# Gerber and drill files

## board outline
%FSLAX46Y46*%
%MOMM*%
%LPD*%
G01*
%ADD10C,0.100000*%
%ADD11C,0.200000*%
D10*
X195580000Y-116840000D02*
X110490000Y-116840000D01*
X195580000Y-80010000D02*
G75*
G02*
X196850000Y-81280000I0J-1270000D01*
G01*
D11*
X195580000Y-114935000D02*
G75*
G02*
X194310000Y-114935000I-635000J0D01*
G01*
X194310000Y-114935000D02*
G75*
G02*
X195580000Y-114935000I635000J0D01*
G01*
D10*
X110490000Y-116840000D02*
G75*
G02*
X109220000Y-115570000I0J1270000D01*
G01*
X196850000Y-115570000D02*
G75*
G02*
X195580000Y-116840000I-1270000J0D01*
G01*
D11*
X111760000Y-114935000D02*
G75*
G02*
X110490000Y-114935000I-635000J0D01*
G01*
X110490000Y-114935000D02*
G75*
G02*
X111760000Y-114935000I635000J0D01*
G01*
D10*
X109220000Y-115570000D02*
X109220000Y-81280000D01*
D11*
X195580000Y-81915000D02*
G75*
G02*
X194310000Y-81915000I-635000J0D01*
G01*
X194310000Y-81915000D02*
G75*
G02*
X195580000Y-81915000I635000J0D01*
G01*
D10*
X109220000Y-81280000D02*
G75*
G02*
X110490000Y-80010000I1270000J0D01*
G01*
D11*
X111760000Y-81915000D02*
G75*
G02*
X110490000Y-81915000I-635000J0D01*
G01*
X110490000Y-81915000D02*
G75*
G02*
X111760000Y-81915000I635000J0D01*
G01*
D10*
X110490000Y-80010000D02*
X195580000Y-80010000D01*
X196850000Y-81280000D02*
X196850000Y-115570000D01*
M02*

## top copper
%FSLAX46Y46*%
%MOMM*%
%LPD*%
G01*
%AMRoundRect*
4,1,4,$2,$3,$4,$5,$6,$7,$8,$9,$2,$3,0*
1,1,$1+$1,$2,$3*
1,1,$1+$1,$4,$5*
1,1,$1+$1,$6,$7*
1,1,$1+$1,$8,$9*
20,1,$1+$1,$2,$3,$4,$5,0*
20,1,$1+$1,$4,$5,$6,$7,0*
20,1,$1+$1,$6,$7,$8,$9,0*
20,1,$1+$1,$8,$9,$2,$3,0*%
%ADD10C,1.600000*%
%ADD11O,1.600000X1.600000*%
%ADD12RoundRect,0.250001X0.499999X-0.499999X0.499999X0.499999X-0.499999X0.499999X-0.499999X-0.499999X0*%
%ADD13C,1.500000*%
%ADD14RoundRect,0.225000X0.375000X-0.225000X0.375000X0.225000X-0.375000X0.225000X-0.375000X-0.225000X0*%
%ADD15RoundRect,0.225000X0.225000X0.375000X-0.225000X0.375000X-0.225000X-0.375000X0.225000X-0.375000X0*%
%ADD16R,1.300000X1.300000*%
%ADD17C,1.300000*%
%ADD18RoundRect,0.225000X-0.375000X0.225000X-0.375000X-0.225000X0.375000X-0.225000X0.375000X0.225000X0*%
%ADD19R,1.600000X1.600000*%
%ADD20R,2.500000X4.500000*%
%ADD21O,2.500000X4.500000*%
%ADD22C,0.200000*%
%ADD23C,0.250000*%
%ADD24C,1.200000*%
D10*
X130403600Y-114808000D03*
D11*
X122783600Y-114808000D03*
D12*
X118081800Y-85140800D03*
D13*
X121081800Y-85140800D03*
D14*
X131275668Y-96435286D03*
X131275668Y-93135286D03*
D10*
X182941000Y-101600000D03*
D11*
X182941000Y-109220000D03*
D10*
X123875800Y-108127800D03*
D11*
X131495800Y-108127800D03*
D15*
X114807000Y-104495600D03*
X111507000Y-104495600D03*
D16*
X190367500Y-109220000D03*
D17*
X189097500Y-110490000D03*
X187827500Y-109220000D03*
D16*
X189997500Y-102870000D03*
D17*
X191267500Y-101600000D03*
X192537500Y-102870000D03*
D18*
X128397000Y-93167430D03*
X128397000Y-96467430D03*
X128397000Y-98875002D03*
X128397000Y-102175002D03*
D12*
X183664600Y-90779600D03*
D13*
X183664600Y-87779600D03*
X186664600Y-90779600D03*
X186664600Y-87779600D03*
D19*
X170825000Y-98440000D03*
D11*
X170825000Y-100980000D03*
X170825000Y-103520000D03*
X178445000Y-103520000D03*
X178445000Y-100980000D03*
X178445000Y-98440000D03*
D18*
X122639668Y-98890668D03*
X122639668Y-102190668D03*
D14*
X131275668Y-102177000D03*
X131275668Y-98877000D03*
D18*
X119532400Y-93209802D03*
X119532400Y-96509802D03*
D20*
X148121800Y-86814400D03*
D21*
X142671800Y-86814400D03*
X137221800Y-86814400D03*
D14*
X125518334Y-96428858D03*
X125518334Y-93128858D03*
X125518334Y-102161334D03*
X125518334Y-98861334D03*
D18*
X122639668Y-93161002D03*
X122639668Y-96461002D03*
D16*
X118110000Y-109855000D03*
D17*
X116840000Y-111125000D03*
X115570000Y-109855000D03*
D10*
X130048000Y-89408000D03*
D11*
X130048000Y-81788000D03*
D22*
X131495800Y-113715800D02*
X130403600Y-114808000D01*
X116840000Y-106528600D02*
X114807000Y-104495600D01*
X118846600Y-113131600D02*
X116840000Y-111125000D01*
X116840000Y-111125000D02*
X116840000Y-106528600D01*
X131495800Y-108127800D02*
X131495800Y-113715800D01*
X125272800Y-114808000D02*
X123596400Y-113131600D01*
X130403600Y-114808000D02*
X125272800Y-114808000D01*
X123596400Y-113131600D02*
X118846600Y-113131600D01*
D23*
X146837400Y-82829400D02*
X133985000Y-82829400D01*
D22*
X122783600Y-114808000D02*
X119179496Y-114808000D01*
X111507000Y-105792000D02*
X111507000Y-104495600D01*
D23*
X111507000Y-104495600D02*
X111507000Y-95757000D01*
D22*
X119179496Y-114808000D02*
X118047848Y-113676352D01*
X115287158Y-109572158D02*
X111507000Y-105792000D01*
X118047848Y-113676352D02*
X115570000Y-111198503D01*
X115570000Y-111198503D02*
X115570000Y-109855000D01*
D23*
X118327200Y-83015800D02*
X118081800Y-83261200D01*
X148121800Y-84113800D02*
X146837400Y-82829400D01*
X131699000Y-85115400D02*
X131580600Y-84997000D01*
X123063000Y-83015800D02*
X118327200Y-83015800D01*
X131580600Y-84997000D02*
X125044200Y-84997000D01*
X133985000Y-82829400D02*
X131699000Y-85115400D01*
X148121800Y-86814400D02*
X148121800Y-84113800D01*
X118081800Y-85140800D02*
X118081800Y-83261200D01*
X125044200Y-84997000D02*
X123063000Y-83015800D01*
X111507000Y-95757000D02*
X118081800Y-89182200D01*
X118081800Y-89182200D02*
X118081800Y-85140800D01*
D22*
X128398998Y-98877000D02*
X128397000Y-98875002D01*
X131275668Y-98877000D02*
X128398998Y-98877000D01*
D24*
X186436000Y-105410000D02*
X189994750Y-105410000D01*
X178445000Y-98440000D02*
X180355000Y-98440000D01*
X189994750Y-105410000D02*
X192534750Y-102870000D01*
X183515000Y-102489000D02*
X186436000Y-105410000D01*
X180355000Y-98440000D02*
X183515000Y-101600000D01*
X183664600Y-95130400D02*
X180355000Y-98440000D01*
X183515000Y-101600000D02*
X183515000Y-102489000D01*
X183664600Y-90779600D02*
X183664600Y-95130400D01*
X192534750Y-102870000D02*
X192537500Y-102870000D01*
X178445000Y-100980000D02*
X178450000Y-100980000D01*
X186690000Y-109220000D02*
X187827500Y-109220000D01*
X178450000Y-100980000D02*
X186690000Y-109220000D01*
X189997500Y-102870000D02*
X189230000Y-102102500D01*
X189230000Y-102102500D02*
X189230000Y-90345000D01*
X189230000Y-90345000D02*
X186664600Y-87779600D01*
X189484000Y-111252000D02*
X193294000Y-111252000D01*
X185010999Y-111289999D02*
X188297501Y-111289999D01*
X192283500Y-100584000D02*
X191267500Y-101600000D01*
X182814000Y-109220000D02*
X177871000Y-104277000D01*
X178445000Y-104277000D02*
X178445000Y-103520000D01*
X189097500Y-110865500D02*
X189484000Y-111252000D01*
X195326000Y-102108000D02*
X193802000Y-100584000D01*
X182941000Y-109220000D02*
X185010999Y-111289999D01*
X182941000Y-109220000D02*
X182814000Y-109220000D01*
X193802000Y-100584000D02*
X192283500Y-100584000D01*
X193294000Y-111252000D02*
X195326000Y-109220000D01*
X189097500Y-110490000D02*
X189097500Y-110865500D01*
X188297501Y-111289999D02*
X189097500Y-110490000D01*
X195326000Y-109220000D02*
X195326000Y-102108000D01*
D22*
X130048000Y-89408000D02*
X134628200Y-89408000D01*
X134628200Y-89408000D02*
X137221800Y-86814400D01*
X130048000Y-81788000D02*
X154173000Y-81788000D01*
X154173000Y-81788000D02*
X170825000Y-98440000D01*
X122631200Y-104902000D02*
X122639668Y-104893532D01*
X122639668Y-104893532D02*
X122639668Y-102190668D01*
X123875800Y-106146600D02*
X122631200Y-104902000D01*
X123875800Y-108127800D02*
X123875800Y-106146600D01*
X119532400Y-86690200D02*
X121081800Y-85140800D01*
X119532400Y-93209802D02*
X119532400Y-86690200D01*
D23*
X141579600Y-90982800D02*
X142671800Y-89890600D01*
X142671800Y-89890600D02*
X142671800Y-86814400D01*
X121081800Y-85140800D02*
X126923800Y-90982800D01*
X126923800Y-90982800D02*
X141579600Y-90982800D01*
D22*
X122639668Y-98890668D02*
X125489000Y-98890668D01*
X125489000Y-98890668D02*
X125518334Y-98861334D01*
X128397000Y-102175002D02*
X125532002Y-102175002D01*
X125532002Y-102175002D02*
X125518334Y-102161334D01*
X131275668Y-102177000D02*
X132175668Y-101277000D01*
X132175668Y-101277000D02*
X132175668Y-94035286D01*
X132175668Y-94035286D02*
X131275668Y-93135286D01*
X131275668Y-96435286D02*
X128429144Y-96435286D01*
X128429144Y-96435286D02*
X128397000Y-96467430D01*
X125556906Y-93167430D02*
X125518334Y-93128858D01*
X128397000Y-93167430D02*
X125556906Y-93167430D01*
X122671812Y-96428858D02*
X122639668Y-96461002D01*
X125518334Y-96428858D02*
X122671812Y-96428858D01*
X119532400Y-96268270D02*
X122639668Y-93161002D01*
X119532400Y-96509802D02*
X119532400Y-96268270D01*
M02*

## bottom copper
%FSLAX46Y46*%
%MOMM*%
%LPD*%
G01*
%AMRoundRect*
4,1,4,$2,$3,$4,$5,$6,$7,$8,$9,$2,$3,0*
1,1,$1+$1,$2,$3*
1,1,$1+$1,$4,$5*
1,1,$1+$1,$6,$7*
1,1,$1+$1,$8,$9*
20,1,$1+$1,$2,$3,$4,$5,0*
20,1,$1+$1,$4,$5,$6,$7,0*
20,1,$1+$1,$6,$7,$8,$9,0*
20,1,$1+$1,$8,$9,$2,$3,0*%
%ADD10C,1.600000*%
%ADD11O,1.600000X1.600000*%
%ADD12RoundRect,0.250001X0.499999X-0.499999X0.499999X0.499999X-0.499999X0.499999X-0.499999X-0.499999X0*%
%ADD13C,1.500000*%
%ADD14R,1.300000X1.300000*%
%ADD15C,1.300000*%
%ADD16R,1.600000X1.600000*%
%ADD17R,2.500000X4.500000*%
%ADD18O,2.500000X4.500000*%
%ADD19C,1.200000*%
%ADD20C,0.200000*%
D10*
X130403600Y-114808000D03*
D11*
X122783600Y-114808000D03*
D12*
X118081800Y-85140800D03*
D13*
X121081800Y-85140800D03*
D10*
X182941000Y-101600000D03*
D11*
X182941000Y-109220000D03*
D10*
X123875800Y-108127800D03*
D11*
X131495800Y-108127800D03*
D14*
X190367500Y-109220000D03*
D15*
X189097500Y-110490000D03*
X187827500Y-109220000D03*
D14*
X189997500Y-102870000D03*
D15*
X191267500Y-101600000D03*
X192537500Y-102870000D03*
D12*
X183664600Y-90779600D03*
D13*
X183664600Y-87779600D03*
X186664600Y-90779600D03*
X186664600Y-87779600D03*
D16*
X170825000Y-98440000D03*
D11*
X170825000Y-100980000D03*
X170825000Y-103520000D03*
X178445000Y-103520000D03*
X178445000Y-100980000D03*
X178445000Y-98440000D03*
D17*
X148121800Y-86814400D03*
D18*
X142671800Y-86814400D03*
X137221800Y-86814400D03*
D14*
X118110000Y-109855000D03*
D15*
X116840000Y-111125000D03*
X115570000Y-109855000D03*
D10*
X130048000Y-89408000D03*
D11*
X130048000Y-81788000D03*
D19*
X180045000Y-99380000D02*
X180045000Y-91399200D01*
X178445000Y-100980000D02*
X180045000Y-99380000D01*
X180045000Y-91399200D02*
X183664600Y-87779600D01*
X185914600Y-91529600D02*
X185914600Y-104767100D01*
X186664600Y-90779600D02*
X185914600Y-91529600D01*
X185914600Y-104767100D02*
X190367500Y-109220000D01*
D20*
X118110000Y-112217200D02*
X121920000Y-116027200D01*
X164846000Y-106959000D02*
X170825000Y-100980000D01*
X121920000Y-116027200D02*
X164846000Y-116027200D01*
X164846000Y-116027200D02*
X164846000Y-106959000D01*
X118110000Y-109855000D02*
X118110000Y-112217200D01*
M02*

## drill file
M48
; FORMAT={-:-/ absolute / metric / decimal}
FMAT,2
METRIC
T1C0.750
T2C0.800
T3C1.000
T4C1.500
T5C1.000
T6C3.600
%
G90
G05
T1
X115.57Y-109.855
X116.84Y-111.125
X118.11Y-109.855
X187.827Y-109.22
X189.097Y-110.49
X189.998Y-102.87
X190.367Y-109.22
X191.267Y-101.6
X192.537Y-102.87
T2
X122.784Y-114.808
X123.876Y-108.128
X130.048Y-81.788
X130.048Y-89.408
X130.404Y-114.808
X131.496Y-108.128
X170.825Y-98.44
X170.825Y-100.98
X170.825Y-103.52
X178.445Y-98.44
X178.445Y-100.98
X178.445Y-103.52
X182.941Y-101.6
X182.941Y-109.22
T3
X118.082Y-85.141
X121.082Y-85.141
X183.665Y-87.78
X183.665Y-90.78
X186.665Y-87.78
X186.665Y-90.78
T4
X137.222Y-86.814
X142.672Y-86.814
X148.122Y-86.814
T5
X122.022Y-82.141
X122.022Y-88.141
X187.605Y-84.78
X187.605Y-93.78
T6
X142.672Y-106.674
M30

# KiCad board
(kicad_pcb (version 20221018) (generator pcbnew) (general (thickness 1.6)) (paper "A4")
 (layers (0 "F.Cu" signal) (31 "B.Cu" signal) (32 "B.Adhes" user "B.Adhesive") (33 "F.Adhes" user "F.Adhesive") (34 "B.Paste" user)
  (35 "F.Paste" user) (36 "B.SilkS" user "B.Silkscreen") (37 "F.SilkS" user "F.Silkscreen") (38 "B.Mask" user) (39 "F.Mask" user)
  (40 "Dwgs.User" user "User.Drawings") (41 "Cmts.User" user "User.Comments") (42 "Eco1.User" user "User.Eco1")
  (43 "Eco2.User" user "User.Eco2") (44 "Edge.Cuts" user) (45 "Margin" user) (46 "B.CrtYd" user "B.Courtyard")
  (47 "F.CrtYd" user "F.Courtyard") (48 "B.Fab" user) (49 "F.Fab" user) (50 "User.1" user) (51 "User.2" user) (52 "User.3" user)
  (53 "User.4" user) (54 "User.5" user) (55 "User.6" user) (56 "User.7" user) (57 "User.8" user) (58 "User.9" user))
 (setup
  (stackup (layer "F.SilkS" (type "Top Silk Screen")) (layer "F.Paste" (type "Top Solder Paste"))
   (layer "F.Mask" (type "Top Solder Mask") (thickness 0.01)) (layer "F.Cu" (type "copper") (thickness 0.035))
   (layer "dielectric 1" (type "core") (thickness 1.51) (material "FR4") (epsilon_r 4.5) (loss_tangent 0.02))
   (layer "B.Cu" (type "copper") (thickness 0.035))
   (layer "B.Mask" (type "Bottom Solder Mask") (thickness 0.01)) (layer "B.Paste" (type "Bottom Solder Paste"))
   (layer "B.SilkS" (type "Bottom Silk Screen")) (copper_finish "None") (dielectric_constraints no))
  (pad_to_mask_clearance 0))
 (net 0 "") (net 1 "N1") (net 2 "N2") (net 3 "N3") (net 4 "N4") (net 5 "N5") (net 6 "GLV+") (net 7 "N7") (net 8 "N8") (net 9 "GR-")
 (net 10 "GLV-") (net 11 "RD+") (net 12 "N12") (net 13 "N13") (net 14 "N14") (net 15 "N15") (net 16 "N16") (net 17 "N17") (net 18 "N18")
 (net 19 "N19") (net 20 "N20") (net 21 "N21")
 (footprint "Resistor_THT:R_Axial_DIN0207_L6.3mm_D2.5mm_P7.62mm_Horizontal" (layer "F.Cu") (at 130.4036 114.808 180)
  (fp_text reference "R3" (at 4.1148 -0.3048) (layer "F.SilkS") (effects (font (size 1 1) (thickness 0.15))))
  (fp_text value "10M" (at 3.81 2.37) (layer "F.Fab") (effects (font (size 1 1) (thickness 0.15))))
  (pad "1" thru_hole circle (at 0 0 180) (size 1.6 1.6) (drill 0.8) (layers "*.Cu" "*.Mask") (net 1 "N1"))
  (pad "2" thru_hole oval (at 7.62 0 180) (size 1.6 1.6) (drill 0.8) (layers "*.Cu" "*.Mask") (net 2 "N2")))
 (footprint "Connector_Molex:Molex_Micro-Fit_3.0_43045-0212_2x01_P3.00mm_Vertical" (layer "F.Cu") (at 118.0818 85.1408 90)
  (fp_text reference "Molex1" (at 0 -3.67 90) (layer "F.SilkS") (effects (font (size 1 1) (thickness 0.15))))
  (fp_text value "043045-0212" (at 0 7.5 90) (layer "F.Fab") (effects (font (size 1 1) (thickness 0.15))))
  (pad "" np_thru_hole circle (at -3 3.94 90) (size 1 1) (drill 1) (layers "*.Cu" "*.Mask"))
  (pad "" np_thru_hole circle (at 3 3.94 90) (size 1 1) (drill 1) (layers "*.Cu" "*.Mask"))
  (pad "1" thru_hole roundrect (at 0 0 90) (size 1.5 1.5) (drill 1) (layers "*.Cu" "*.Mask") (roundrect_rratio 0.166667) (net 2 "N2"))
  (pad "2" thru_hole circle (at 0 3 90) (size 1.5 1.5) (drill 1) (layers "*.Cu" "*.Mask") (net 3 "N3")))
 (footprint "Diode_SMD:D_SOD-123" (layer "F.Cu") (at 131.275668 94.785286 90)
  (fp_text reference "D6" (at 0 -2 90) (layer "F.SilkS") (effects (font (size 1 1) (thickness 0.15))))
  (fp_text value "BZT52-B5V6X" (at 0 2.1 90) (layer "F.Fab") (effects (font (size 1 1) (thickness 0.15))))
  (pad "1" smd roundrect (at -1.65 0 90) (size 0.9 1.2) (layers "F.Cu" "F.Paste" "F.Mask") (roundrect_rratio 0.25) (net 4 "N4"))
  (pad "2" smd roundrect (at 1.65 0 90) (size 0.9 1.2) (layers "F.Cu" "F.Paste" "F.Mask") (roundrect_rratio 0.25) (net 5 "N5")))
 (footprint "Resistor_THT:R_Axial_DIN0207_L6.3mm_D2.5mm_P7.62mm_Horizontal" (layer "F.Cu") (at 182.941 101.6 -90)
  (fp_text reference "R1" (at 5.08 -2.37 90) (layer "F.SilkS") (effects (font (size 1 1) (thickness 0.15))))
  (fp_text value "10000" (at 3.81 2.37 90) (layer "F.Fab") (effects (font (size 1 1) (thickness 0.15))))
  (pad "1" thru_hole circle (at 0 0 270) (size 1.6 1.6) (drill 0.8) (layers "*.Cu" "*.Mask") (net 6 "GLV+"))
  (pad "2" thru_hole oval (at 7.62 0 270) (size 1.6 1.6) (drill 0.8) (layers "*.Cu" "*.Mask") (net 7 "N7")))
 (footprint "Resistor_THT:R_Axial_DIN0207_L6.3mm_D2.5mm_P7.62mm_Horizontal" (layer "F.Cu") (at 123.8758 108.1278)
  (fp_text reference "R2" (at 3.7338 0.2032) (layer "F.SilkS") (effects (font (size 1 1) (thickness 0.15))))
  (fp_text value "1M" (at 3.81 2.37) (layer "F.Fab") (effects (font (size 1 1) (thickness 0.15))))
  (pad "1" thru_hole circle (at 0 0) (size 1.6 1.6) (drill 0.8) (layers "*.Cu" "*.Mask") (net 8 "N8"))
  (pad "2" thru_hole oval (at 7.62 0) (size 1.6 1.6) (drill 0.8) (layers "*.Cu" "*.Mask") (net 1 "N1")))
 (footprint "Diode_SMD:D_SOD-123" (layer "F.Cu") (at 113.157 104.4956 180)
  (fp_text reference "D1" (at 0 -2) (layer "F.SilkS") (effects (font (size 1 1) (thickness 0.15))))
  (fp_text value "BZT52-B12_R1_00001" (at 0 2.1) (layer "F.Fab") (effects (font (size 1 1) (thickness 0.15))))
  (pad "1" smd roundrect (at -1.65 0 180) (size 0.9 1.2) (layers "F.Cu" "F.Paste" "F.Mask") (roundrect_rratio 0.25) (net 1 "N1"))
  (pad "2" smd roundrect (at 1.65 0 180) (size 0.9 1.2) (layers "F.Cu" "F.Paste" "F.Mask") (roundrect_rratio 0.25) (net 2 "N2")))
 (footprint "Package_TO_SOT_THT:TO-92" (layer "F.Cu") (at 190.3675 109.22 180)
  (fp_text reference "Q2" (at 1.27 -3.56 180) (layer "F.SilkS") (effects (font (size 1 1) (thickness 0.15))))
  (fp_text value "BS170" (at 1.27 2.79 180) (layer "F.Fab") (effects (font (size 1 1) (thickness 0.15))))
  (pad "1" thru_hole rect (at 0 0 180) (size 1.3 1.3) (drill 0.75) (layers "*.Cu" "*.Mask") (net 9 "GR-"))
  (pad "2" thru_hole circle (at 1.27 -1.27 180) (size 1.3 1.3) (drill 0.75) (layers "*.Cu" "*.Mask") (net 7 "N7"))
  (pad "3" thru_hole circle (at 2.54 0 180) (size 1.3 1.3) (drill 0.75) (layers "*.Cu" "*.Mask") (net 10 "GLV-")))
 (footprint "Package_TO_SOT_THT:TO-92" (layer "F.Cu") (at 189.9975 102.87)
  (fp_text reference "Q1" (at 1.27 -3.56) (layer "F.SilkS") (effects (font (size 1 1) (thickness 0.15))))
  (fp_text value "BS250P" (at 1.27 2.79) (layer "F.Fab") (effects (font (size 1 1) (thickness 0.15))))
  (pad "1" thru_hole rect (at 0 0) (size 1.3 1.3) (drill 0.75) (layers "*.Cu" "*.Mask") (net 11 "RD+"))
  (pad "2" thru_hole circle (at 1.27 -1.27) (size 1.3 1.3) (drill 0.75) (layers "*.Cu" "*.Mask") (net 7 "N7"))
  (pad "3" thru_hole circle (at 2.54 0) (size 1.3 1.3) (drill 0.75) (layers "*.Cu" "*.Mask") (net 6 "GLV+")))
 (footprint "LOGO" (layer "F.Cu") (at 157.988 103.124)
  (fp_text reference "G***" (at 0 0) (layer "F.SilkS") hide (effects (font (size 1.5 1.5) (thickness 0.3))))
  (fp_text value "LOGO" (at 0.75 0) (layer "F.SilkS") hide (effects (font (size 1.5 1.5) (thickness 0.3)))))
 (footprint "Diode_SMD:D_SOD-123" (layer "F.Cu") (at 128.397 94.81743 -90)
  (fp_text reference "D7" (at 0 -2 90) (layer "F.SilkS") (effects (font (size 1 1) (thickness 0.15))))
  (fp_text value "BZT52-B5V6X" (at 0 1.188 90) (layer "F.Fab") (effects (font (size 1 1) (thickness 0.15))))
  (pad "1" smd roundrect (at -1.65 0 270) (size 0.9 1.2) (layers "F.Cu" "F.Paste" "F.Mask") (roundrect_rratio 0.25) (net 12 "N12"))
  (pad "2" smd roundrect (at 1.65 0 270) (size 0.9 1.2) (layers "F.Cu" "F.Paste" "F.Mask") (roundrect_rratio 0.25) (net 4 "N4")))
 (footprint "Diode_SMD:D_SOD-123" (layer "F.Cu") (at 128.397 100.525002 -90)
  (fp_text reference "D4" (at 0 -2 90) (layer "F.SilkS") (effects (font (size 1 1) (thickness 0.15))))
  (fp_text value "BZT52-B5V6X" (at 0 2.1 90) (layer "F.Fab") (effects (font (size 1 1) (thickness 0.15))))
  (pad "1" smd roundrect (at -1.65 0 270) (size 0.9 1.2) (layers "F.Cu" "F.Paste" "F.Mask") (roundrect_rratio 0.25) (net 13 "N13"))
  (pad "2" smd roundrect (at 1.65 0 270) (size 0.9 1.2) (layers "F.Cu" "F.Paste" "F.Mask") (roundrect_rratio 0.25) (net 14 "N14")))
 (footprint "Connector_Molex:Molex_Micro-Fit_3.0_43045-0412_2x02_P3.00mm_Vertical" (layer "F.Cu") (at 183.6646 90.7796 90)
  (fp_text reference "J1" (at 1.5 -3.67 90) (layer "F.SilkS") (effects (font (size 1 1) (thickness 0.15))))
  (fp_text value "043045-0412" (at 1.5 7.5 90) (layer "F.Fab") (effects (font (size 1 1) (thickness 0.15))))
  (pad "" np_thru_hole circle (at -3 3.94 90) (size 1 1) (drill 1) (layers "*.Cu" "*.Mask"))
  (pad "" np_thru_hole circle (at 6 3.94 90) (size 1 1) (drill 1) (layers "*.Cu" "*.Mask"))
  (pad "1" thru_hole roundrect (at 0 0 90) (size 1.5 1.5) (drill 1) (layers "*.Cu" "*.Mask") (roundrect_rratio 0.166667) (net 6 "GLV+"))
  (pad "2" thru_hole circle (at 3 0 90) (size 1.5 1.5) (drill 1) (layers "*.Cu" "*.Mask") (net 10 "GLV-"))
  (pad "3" thru_hole circle (at 0 3 90) (size 1.5 1.5) (drill 1) (layers "*.Cu" "*.Mask") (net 9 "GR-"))
  (pad "4" thru_hole circle (at 3 3 90) (size 1.5 1.5) (drill 1) (layers "*.Cu" "*.Mask") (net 11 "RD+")))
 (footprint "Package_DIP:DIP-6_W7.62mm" (layer "F.Cu") (at 170.825 98.44)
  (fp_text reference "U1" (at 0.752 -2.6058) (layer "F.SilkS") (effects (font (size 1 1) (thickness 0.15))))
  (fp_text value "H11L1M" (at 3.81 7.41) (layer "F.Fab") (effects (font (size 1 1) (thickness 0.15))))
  (pad "1" thru_hole rect (at 0 0) (size 1.6 1.6) (drill 0.8) (layers "*.Cu" "*.Mask") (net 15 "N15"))
  (pad "2" thru_hole oval (at 0 2.54) (size 1.6 1.6) (drill 0.8) (layers "*.Cu" "*.Mask") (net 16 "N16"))
  (pad "3" thru_hole oval (at 0 5.08) (size 1.6 1.6) (drill 0.8) (layers "*.Cu" "*.Mask") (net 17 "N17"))
  (pad "4" thru_hole oval (at 7.62 5.08) (size 1.6 1.6) (drill 0.8) (layers "*.Cu" "*.Mask") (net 7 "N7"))
  (pad "5" thru_hole oval (at 7.62 2.54) (size 1.6 1.6) (drill 0.8) (layers "*.Cu" "*.Mask") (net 10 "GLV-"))
  (pad "6" thru_hole oval (at 7.62 0) (size 1.6 1.6) (drill 0.8) (layers "*.Cu" "*.Mask") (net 6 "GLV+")))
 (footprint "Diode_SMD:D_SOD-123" (layer "F.Cu") (at 122.639668 100.540668 -90)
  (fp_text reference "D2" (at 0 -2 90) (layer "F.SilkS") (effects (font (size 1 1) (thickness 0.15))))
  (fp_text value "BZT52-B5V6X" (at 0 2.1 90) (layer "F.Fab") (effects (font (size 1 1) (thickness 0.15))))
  (pad "1" smd roundrect (at -1.65 0 270) (size 0.9 1.2) (layers "F.Cu" "F.Paste" "F.Mask") (roundrect_rratio 0.25) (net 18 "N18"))
  (pad "2" smd roundrect (at 1.65 0 270) (size 0.9 1.2) (layers "F.Cu" "F.Paste" "F.Mask") (roundrect_rratio 0.25) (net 8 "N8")))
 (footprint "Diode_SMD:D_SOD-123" (layer "F.Cu") (at 131.275668 100.527 90)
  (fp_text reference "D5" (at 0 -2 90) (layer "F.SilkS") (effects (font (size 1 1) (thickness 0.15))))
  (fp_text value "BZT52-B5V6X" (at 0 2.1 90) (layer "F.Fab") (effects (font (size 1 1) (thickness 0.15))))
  (pad "1" smd roundrect (at -1.65 0 90) (size 0.9 1.2) (layers "F.Cu" "F.Paste" "F.Mask") (roundrect_rratio 0.25) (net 5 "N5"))
  (pad "2" smd roundrect (at 1.65 0 90) (size 0.9 1.2) (layers "F.Cu" "F.Paste" "F.Mask") (roundrect_rratio 0.25) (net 13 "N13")))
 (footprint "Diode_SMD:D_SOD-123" (layer "F.Cu") (at 119.5324 94.859802 -90)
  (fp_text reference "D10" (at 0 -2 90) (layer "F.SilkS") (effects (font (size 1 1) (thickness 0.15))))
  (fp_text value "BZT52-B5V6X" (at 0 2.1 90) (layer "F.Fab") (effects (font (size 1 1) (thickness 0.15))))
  (pad "1" smd roundrect (at -1.65 0 270) (size 0.9 1.2) (layers "F.Cu" "F.Paste" "F.Mask") (roundrect_rratio 0.25) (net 3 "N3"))
  (pad "2" smd roundrect (at 1.65 0 270) (size 0.9 1.2) (layers "F.Cu" "F.Paste" "F.Mask") (roundrect_rratio 0.25) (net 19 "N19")))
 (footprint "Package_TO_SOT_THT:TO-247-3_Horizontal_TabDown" (layer "F.Cu") (at 148.1218 86.8144 180)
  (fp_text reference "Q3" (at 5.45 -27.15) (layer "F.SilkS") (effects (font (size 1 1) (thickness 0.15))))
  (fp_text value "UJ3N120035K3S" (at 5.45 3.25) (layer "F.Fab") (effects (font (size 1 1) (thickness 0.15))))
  (pad "" np_thru_hole oval (at 5.45 -19.86 180) (size 3.6 3.6) (drill 3.6) (layers "*.Cu" "*.Mask"))
  (pad "1" thru_hole rect (at 0 0 180) (size 2.5 4.5) (drill 1.5) (layers "*.Cu" "*.Mask") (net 2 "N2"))
  (pad "2" thru_hole oval (at 5.45 0 180) (size 2.5 4.5) (drill 1.5) (layers "*.Cu" "*.Mask") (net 3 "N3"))
  (pad "3" thru_hole oval (at 10.9 0 180) (size 2.5 4.5) (drill 1.5) (layers "*.Cu" "*.Mask") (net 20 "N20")))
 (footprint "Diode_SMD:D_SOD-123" (layer "F.Cu") (at 125.518334 94.778858 90)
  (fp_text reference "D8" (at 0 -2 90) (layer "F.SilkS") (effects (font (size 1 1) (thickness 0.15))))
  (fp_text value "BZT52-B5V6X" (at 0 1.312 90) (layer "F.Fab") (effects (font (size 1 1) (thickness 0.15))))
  (pad "1" smd roundrect (at -1.65 0 90) (size 0.9 1.2) (layers "F.Cu" "F.Paste" "F.Mask") (roundrect_rratio 0.25) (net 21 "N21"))
  (pad "2" smd roundrect (at 1.65 0 90) (size 0.9 1.2) (layers "F.Cu" "F.Paste" "F.Mask") (roundrect_rratio 0.25) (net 12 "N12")))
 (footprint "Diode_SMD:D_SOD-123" (layer "F.Cu") (at 125.518334 100.511334 90)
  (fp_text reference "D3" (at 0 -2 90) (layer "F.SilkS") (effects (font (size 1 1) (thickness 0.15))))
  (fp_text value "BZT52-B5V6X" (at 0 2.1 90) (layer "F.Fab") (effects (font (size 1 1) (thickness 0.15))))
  (pad "1" smd roundrect (at -1.65 0 90) (size 0.9 1.2) (layers "F.Cu" "F.Paste" "F.Mask") (roundrect_rratio 0.25) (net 14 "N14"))
  (pad "2" smd roundrect (at 1.65 0 90) (size 0.9 1.2) (layers "F.Cu" "F.Paste" "F.Mask") (roundrect_rratio 0.25) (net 18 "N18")))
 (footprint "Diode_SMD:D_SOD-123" (layer "F.Cu") (at 122.639668 94.811002 -90)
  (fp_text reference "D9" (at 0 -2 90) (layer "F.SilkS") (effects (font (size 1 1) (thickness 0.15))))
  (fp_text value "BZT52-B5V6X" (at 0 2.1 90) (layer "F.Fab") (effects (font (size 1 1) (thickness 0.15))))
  (pad "1" smd roundrect (at -1.65 0 270) (size 0.9 1.2) (layers "F.Cu" "F.Paste" "F.Mask") (roundrect_rratio 0.25) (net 19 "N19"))
  (pad "2" smd roundrect (at 1.65 0 270) (size 0.9 1.2) (layers "F.Cu" "F.Paste" "F.Mask") (roundrect_rratio 0.25) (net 21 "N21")))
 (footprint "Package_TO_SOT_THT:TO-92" (layer "F.Cu") (at 118.11 109.855 180)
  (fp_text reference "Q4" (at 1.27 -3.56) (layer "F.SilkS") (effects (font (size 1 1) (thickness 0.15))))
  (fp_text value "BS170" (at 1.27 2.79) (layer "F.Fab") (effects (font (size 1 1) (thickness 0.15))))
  (pad "1" thru_hole rect (at 0 0 180) (size 1.3 1.3) (drill 0.75) (layers "*.Cu" "*.Mask") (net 16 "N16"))
  (pad "2" thru_hole circle (at 1.27 -1.27 180) (size 1.3 1.3) (drill 0.75) (layers "*.Cu" "*.Mask") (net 1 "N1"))
  (pad "3" thru_hole circle (at 2.54 0 180) (size 1.3 1.3) (drill 0.75) (layers "*.Cu" "*.Mask") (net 2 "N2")))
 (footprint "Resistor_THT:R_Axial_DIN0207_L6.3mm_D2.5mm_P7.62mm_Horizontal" (layer "F.Cu") (at 130.048 89.408 90)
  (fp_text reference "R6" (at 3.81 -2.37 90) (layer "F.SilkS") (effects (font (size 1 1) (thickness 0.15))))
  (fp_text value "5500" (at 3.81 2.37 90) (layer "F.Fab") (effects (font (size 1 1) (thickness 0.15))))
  (pad "1" thru_hole circle (at 0 0 90) (size 1.6 1.6) (drill 0.8) (layers "*.Cu" "*.Mask") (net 20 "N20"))
  (pad "2" thru_hole oval (at 7.62 0 90) (size 1.6 1.6) (drill 0.8) (layers "*.Cu" "*.Mask") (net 15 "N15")))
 (gr_line (start 195.58 116.84) (end 110.49 116.84) (stroke (width 0.1) (type default)) (layer "Edge.Cuts"))
 (gr_arc (start 195.58 80.01) (mid 196.478026 80.381974) (end 196.85 81.28) (stroke (width 0.1) (type default)) (layer "Edge.Cuts"))
 (gr_circle (center 194.945 114.935) (end 195.58 114.935) (stroke (width 0.2) (type default)) (fill none) (layer "Edge.Cuts"))
 (gr_arc (start 110.49 116.84) (mid 109.591974 116.468026) (end 109.22 115.57) (stroke (width 0.1) (type default)) (layer "Edge.Cuts"))
 (gr_arc (start 196.85 115.57) (mid 196.478026 116.468026) (end 195.58 116.84) (stroke (width 0.1) (type default)) (layer "Edge.Cuts"))
 (gr_circle (center 111.125 114.935) (end 111.76 114.935) (stroke (width 0.2) (type default)) (fill none) (layer "Edge.Cuts"))
 (gr_line (start 109.22 115.57) (end 109.22 81.28) (stroke (width 0.1) (type default)) (layer "Edge.Cuts"))
 (gr_circle (center 194.945 81.915) (end 195.58 81.915) (stroke (width 0.2) (type default)) (fill none) (layer "Edge.Cuts"))
 (gr_arc (start 109.22 81.28) (mid 109.591974 80.381974) (end 110.49 80.01) (stroke (width 0.1) (type default)) (layer "Edge.Cuts"))
 (gr_circle (center 111.125 81.915) (end 111.76 81.915) (stroke (width 0.2) (type default)) (fill none) (layer "Edge.Cuts"))
 (gr_line (start 110.49 80.01) (end 195.58 80.01) (stroke (width 0.1) (type default)) (layer "Edge.Cuts"))
 (gr_line (start 196.85 81.28) (end 196.85 115.57) (stroke (width 0.1) (type default)) (layer "Edge.Cuts"))
 (segment (start 131.4958 113.7158) (end 130.4036 114.808) (width 0.2) (layer "F.Cu") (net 1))
 (segment (start 116.84 106.5286) (end 114.807 104.4956) (width 0.2) (layer "F.Cu") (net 1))
 (segment (start 118.8466 113.1316) (end 116.84 111.125) (width 0.2) (layer "F.Cu") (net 1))
 (segment (start 116.84 111.125) (end 116.84 106.5286) (width 0.2) (layer "F.Cu") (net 1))
 (segment (start 131.4958 108.1278) (end 131.4958 113.7158) (width 0.2) (layer "F.Cu") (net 1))
 (segment (start 125.2728 114.808) (end 123.5964 113.1316) (width 0.2) (layer "F.Cu") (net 1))
 (segment (start 130.4036 114.808) (end 125.2728 114.808) (width 0.2) (layer "F.Cu") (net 1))
 (segment (start 123.5964 113.1316) (end 118.8466 113.1316) (width 0.2) (layer "F.Cu") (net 1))
 (segment (start 146.8374 82.8294) (end 133.985 82.8294) (width 0.25) (layer "F.Cu") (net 2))
 (segment (start 122.7836 114.808) (end 119.179496 114.808) (width 0.2) (layer "F.Cu") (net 2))
 (segment (start 111.507 105.792) (end 111.507 104.4956) (width 0.2) (layer "F.Cu") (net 2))
 (segment (start 111.507 104.4956) (end 111.507 95.757) (width 0.25) (layer "F.Cu") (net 2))
 (segment (start 119.179496 114.808) (end 118.047848 113.676352) (width 0.2) (layer "F.Cu") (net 2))
 (segment (start 115.287158 109.572158) (end 111.507 105.792) (width 0.2) (layer "F.Cu") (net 2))
 (segment (start 118.047848 113.676352) (end 115.57 111.198503) (width 0.2) (layer "F.Cu") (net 2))
 (segment (start 115.57 111.198503) (end 115.57 109.855) (width 0.2) (layer "F.Cu") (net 2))
 (segment (start 118.3272 83.0158) (end 118.0818 83.2612) (width 0.25) (layer "F.Cu") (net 2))
 (segment (start 148.1218 84.1138) (end 146.8374 82.8294) (width 0.25) (layer "F.Cu") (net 2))
 (segment (start 131.699 85.1154) (end 131.5806 84.997) (width 0.25) (layer "F.Cu") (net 2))
 (segment (start 123.063 83.0158) (end 118.3272 83.0158) (width 0.25) (layer "F.Cu") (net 2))
 (segment (start 131.5806 84.997) (end 125.0442 84.997) (width 0.25) (layer "F.Cu") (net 2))
 (segment (start 133.985 82.8294) (end 131.699 85.1154) (width 0.25) (layer "F.Cu") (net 2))
 (segment (start 148.1218 86.8144) (end 148.1218 84.1138) (width 0.25) (layer "F.Cu") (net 2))
 (segment (start 118.0818 85.1408) (end 118.0818 83.2612) (width 0.25) (layer "F.Cu") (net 2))
 (segment (start 125.0442 84.997) (end 123.063 83.0158) (width 0.25) (layer "F.Cu") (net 2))
 (segment (start 111.507 95.757) (end 118.0818 89.1822) (width 0.25) (layer "F.Cu") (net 2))
 (segment (start 118.0818 89.1822) (end 118.0818 85.1408) (width 0.25) (layer "F.Cu") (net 2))
 (segment (start 128.398998 98.877) (end 128.397 98.875002) (width 0.2) (layer "F.Cu") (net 13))
 (segment (start 131.275668 98.877) (end 128.398998 98.877) (width 0.2) (layer "F.Cu") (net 13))
 (segment (start 186.436 105.41) (end 189.99475 105.41) (width 1.2) (layer "F.Cu") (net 6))
 (segment (start 178.445 98.44) (end 180.355 98.44) (width 1.2) (layer "F.Cu") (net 6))
 (segment (start 189.99475 105.41) (end 192.53475 102.87) (width 1.2) (layer "F.Cu") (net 6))
 (segment (start 183.515 102.489) (end 186.436 105.41) (width 1.2) (layer "F.Cu") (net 6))
 (segment (start 180.355 98.44) (end 183.515 101.6) (width 1.2) (layer "F.Cu") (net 6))
 (segment (start 183.6646 95.1304) (end 180.355 98.44) (width 1.2) (layer "F.Cu") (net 6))
 (segment (start 183.515 101.6) (end 183.515 102.489) (width 1.2) (layer "F.Cu") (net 6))
 (segment (start 183.6646 90.7796) (end 183.6646 95.1304) (width 1.2) (layer "F.Cu") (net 6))
 (segment (start 192.53475 102.87) (end 192.5375 102.87) (width 1.2) (layer "F.Cu") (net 6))
 (segment (start 178.445 100.98) (end 178.45 100.98) (width 1.2) (layer "F.Cu") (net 10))
 (segment (start 186.69 109.22) (end 187.8275 109.22) (width 1.2) (layer "F.Cu") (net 10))
 (segment (start 178.45 100.98) (end 186.69 109.22) (width 1.2) (layer "F.Cu") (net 10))
 (segment (start 180.045 99.38) (end 180.045 91.3992) (width 1.2) (layer "B.Cu") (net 10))
 (segment (start 178.445 100.98) (end 180.045 99.38) (width 1.2) (layer "B.Cu") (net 10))
 (segment (start 180.045 91.3992) (end 183.6646 87.7796) (width 1.2) (layer "B.Cu") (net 10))
 (segment (start 185.9146 91.5296) (end 185.9146 104.7671) (width 1.2) (layer "B.Cu") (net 9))
 (segment (start 186.6646 90.7796) (end 185.9146 91.5296) (width 1.2) (layer "B.Cu") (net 9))
 (segment (start 185.9146 104.7671) (end 190.3675 109.22) (width 1.2) (layer "B.Cu") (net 9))
 (segment (start 189.9975 102.87) (end 189.23 102.1025) (width 1.2) (layer "F.Cu") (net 11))
 (segment (start 189.23 102.1025) (end 189.23 90.345) (width 1.2) (layer "F.Cu") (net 11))
 (segment (start 189.23 90.345) (end 186.6646 87.7796) (width 1.2) (layer "F.Cu") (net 11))
 (segment (start 189.484 111.252) (end 193.294 111.252) (width 1.2) (layer "F.Cu") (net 7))
 (segment (start 185.010999 111.289999) (end 188.297501 111.289999) (width 1.2) (layer "F.Cu") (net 7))
 (segment (start 192.2835 100.584) (end 191.2675 101.6) (width 1.2) (layer "F.Cu") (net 7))
 (segment (start 182.814 109.22) (end 177.871 104.277) (width 1.2) (layer "F.Cu") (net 7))
 (segment (start 178.445 104.277) (end 178.445 103.52) (width 1.2) (layer "F.Cu") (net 7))
 (segment (start 189.0975 110.8655) (end 189.484 111.252) (width 1.2) (layer "F.Cu") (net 7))
 (segment (start 195.326 102.108) (end 193.802 100.584) (width 1.2) (layer "F.Cu") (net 7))
 (segment (start 182.941 109.22) (end 185.010999 111.289999) (width 1.2) (layer "F.Cu") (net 7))
 (segment (start 182.941 109.22) (end 182.814 109.22) (width 1.2) (layer "F.Cu") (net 7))
 (segment (start 193.802 100.584) (end 192.2835 100.584) (width 1.2) (layer "F.Cu") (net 7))
 (segment (start 193.294 111.252) (end 195.326 109.22) (width 1.2) (layer "F.Cu") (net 7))
 (segment (start 189.0975 110.49) (end 189.0975 110.8655) (width 1.2) (layer "F.Cu") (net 7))
 (segment (start 188.297501 111.289999) (end 189.0975 110.49) (width 1.2) (layer "F.Cu") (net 7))
 (segment (start 195.326 109.22) (end 195.326 102.108) (width 1.2) (layer "F.Cu") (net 7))
 (segment (start 130.048 89.408) (end 134.6282 89.408) (width 0.2) (layer "F.Cu") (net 20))
 (segment (start 134.6282 89.408) (end 137.2218 86.8144) (width 0.2) (layer "F.Cu") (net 20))
 (segment (start 118.11 112.2172) (end 121.92 116.0272) (width 0.2) (layer "B.Cu") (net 16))
 (segment (start 164.846 106.959) (end 170.825 100.98) (width 0.2) (layer "B.Cu") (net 16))
 (segment (start 121.92 116.0272) (end 164.846 116.0272) (width 0.2) (layer "B.Cu") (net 16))
 (segment (start 164.846 116.0272) (end 164.846 106.959) (width 0.2) (layer "B.Cu") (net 16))
 (segment (start 118.11 109.855) (end 118.11 112.2172) (width 0.2) (layer "B.Cu") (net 16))
 (segment (start 130.048 81.788) (end 154.173 81.788) (width 0.2) (layer "F.Cu") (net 15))
 (segment (start 154.173 81.788) (end 170.825 98.44) (width 0.2) (layer "F.Cu") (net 15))
 (segment (start 122.6312 104.902) (end 122.639668 104.893532) (width 0.2) (layer "F.Cu") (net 8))
 (segment (start 122.639668 104.893532) (end 122.639668 102.190668) (width 0.2) (layer "F.Cu") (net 8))
 (segment (start 123.8758 106.1466) (end 122.6312 104.902) (width 0.2) (layer "F.Cu") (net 8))
 (segment (start 123.8758 108.1278) (end 123.8758 106.1466) (width 0.2) (layer "F.Cu") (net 8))
 (segment (start 119.5324 86.6902) (end 121.0818 85.1408) (width 0.2) (layer "F.Cu") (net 3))
 (segment (start 119.5324 93.209802) (end 119.5324 86.6902) (width 0.2) (layer "F.Cu") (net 3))
 (segment (start 141.5796 90.9828) (end 142.6718 89.8906) (width 0.25) (layer "F.Cu") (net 3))
 (segment (start 142.6718 89.8906) (end 142.6718 86.8144) (width 0.25) (layer "F.Cu") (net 3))
 (segment (start 121.0818 85.1408) (end 126.9238 90.9828) (width 0.25) (layer "F.Cu") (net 3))
 (segment (start 126.9238 90.9828) (end 141.5796 90.9828) (width 0.25) (layer "F.Cu") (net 3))
 (segment (start 122.639668 98.890668) (end 125.489 98.890668) (width 0.2) (layer "F.Cu") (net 18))
 (segment (start 125.489 98.890668) (end 125.518334 98.861334) (width 0.2) (layer "F.Cu") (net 18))
 (segment (start 128.397 102.175002) (end 125.532002 102.175002) (width 0.2) (layer "F.Cu") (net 14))
 (segment (start 125.532002 102.175002) (end 125.518334 102.161334) (width 0.2) (layer "F.Cu") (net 14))
 (segment (start 131.275668 102.177) (end 132.175668 101.277) (width 0.2) (layer "F.Cu") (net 5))
 (segment (start 132.175668 101.277) (end 132.175668 94.035286) (width 0.2) (layer "F.Cu") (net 5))
 (segment (start 132.175668 94.035286) (end 131.275668 93.135286) (width 0.2) (layer "F.Cu") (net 5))
 (segment (start 131.275668 96.435286) (end 128.429144 96.435286) (width 0.2) (layer "F.Cu") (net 4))
 (segment (start 128.429144 96.435286) (end 128.397 96.46743) (width 0.2) (layer "F.Cu") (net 4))
 (segment (start 125.556906 93.16743) (end 125.518334 93.128858) (width 0.2) (layer "F.Cu") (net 12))
 (segment (start 128.397 93.16743) (end 125.556906 93.16743) (width 0.2) (layer "F.Cu") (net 12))
 (segment (start 122.671812 96.428858) (end 122.639668 96.461002) (width 0.2) (layer "F.Cu") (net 21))
 (segment (start 125.518334 96.428858) (end 122.671812 96.428858) (width 0.2) (layer "F.Cu") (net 21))
 (segment (start 119.5324 96.26827) (end 122.639668 93.161002) (width 0.2) (layer "F.Cu") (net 19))
 (segment (start 119.5324 96.509802) (end 119.5324 96.26827) (width 0.2) (layer "F.Cu") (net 19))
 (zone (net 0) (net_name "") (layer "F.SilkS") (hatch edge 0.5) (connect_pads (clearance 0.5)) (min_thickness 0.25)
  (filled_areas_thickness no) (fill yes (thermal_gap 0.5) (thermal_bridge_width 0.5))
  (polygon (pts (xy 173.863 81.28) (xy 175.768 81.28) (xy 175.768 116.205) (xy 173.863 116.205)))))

